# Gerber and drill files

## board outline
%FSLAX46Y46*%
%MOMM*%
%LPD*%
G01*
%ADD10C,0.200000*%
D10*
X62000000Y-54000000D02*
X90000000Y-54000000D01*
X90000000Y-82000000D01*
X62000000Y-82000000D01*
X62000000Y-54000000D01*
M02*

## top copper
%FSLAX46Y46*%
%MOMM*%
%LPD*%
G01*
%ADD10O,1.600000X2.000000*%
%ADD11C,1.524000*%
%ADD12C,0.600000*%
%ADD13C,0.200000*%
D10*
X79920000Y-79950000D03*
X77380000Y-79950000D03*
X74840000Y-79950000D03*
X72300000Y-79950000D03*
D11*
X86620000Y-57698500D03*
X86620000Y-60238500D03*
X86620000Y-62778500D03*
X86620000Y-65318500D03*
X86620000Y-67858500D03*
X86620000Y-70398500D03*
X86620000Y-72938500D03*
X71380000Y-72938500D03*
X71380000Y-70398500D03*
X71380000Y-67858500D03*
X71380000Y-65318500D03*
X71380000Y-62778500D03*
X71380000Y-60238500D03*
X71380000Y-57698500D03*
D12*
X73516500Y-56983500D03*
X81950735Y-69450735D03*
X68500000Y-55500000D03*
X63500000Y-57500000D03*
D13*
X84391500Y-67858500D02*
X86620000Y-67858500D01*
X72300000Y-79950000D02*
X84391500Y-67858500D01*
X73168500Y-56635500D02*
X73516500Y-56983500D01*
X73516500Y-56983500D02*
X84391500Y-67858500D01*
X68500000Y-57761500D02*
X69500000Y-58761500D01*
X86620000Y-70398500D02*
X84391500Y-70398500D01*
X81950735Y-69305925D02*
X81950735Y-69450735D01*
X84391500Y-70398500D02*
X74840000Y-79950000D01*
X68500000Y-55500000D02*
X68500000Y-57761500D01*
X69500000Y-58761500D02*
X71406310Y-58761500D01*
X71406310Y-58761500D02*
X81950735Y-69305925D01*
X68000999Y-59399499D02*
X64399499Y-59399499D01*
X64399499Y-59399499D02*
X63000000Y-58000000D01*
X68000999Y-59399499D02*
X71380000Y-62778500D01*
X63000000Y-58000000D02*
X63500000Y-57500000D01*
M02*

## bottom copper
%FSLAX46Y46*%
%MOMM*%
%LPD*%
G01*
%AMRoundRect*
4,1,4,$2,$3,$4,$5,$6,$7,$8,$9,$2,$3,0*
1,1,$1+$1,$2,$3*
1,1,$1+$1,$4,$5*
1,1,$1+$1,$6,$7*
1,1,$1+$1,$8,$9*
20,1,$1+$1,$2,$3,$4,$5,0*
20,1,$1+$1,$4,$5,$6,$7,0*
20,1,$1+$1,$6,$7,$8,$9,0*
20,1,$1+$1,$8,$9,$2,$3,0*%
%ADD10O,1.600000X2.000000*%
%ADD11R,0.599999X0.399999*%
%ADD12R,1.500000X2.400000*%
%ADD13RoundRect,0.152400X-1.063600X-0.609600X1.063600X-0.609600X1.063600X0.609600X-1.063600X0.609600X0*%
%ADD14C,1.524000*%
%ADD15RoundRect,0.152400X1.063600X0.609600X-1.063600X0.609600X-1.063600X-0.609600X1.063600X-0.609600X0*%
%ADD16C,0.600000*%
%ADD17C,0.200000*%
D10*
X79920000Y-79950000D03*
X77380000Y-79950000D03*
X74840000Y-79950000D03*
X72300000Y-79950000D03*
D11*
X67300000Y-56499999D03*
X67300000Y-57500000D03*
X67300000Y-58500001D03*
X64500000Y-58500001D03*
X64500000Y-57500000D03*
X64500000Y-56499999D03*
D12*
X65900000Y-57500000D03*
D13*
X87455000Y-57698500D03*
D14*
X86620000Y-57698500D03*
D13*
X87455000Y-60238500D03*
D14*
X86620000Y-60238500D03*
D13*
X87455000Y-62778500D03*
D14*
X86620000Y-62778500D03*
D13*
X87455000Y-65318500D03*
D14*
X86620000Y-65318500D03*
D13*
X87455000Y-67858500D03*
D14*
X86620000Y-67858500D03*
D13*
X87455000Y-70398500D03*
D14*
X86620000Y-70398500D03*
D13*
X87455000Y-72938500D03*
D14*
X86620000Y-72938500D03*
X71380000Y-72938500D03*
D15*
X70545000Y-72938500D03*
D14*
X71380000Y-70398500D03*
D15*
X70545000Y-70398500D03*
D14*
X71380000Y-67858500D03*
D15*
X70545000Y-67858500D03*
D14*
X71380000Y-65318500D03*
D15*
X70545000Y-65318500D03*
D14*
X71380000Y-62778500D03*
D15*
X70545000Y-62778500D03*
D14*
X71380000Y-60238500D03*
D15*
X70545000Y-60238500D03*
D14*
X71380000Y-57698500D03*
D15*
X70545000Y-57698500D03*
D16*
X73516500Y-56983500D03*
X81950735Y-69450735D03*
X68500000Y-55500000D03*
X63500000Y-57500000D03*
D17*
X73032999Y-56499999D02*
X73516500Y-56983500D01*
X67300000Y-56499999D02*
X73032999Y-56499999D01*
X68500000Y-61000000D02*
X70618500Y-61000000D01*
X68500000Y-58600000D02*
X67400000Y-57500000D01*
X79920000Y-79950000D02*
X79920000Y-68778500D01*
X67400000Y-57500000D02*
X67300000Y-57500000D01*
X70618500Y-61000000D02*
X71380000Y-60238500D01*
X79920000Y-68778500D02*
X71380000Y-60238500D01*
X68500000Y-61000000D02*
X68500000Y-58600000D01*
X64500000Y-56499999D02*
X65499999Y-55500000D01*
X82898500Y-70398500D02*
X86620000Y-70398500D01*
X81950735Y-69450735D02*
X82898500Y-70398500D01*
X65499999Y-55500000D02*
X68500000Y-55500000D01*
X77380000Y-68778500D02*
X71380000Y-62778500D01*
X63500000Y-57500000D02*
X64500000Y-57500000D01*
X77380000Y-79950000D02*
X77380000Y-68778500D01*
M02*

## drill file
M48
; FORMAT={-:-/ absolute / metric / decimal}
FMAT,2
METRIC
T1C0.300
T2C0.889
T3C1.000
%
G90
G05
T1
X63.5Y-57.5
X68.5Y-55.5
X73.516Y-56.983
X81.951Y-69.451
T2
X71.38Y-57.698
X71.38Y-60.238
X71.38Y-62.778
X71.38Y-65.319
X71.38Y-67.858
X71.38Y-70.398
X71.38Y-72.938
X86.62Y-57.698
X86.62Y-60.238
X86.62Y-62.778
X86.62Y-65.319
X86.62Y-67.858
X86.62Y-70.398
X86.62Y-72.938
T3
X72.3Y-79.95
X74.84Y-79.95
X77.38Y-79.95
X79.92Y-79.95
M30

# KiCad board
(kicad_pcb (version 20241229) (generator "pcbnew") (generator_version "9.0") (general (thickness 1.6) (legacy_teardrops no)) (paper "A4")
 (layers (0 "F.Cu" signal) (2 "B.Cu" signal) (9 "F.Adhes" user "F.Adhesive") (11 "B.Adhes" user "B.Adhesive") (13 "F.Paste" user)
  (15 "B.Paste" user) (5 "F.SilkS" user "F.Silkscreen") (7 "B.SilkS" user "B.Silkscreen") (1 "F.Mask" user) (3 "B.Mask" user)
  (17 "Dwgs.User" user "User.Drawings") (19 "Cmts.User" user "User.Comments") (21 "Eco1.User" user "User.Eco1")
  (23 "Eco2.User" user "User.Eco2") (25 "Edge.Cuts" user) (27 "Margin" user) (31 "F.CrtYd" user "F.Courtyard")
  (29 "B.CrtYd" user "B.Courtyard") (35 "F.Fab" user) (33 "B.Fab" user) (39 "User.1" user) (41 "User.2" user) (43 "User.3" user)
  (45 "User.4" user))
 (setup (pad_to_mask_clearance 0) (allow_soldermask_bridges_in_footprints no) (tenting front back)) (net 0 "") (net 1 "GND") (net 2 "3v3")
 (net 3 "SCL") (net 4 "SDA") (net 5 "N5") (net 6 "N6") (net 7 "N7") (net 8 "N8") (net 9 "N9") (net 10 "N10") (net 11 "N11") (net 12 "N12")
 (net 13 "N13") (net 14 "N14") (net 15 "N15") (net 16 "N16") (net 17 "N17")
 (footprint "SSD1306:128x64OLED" (layer "F.Cu") (at 76.3 69.35 180)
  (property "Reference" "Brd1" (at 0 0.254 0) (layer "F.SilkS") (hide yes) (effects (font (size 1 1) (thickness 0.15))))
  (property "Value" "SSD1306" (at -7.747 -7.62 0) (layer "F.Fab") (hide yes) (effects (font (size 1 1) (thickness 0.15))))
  (pad "1" thru_hole oval (at -3.62 -10.6 270) (size 2 1.6) (drill 1) (layers "*.Cu" "*.Mask") (remove_unused_layers no) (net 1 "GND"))
  (pad "2" thru_hole oval (at -1.08 -10.6 270) (size 2 1.6) (drill 1) (layers "*.Cu" "*.Mask") (remove_unused_layers no) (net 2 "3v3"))
  (pad "3" thru_hole oval (at 1.46 -10.6 270) (size 2 1.6) (drill 1) (layers "*.Cu" "*.Mask") (remove_unused_layers no) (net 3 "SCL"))
  (pad "4" thru_hole oval (at 4 -10.6 270) (size 2 1.6) (drill 1) (layers "*.Cu" "*.Mask") (remove_unused_layers no) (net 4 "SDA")))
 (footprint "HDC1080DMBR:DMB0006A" (layer "B.Cu") (at 65.9 57.5 180)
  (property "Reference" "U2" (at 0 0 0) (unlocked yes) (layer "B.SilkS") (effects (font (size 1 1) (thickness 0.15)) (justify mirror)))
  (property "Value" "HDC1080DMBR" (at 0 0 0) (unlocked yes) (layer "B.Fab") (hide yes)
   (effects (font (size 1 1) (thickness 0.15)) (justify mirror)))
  (pad "1" smd rect (at -1.4 1.000001 180) (size 0.599999 0.399999) (layers "B.Cu" "B.Mask" "B.Paste") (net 4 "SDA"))
  (pad "2" smd rect (at -1.4 0 180) (size 0.599999 0.399999) (layers "B.Cu" "B.Mask" "B.Paste") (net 1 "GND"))
  (pad "3" smd rect (at -1.4 -1.000001 180) (size 0.599999 0.399999) (layers "B.Cu" "B.Mask" "B.Paste") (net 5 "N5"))
  (pad "4" smd rect (at 1.4 -1.000001 180) (size 0.599999 0.399999) (layers "B.Cu" "B.Mask" "B.Paste") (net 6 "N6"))
  (pad "5" smd rect (at 1.4 0 180) (size 0.599999 0.399999) (layers "B.Cu" "B.Mask" "B.Paste") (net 2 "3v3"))
  (pad "6" smd rect (at 1.4 1.000001 180) (size 0.599999 0.399999) (layers "B.Cu" "B.Mask" "B.Paste") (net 3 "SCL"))
  (pad "7" smd rect (at 0 0 180) (size 1.5 2.4) (layers "B.Cu" "B.Mask") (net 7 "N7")))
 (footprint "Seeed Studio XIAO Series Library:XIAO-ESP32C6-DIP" (layer "B.Cu") (at 78.955 65.3185 180)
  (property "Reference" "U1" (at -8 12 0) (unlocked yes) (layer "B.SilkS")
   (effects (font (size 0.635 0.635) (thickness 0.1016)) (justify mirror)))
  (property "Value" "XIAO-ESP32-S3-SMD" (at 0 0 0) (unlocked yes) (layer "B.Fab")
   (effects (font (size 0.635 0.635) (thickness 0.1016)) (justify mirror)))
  (pad "1" smd roundrect (at -8.5 7.62) (size 2.432 1.524) (layers "B.Cu" "B.Mask") (roundrect_rratio 0.1) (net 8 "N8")
   (thermal_bridge_angle 45))
  (pad "1" thru_hole circle (at -7.665 7.62) (size 1.524 1.524) (drill 0.889) (layers "*.Cu" "*.Mask") (remove_unused_layers no)
   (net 8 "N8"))
  (pad "2" smd roundrect (at -8.5 5.08) (size 2.432 1.524) (layers "B.Cu" "B.Mask") (roundrect_rratio 0.1) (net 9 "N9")
   (thermal_bridge_angle 45))
  (pad "2" thru_hole circle (at -7.665 5.08) (size 1.524 1.524) (drill 0.889) (layers "*.Cu" "*.Mask") (remove_unused_layers no)
   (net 9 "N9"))
  (pad "3" smd roundrect (at -8.5 2.54) (size 2.432 1.524) (layers "B.Cu" "B.Mask") (roundrect_rratio 0.1) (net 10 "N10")
   (thermal_bridge_angle 45))
  (pad "3" thru_hole circle (at -7.665 2.54) (size 1.524 1.524) (drill 0.889) (layers "*.Cu" "*.Mask") (remove_unused_layers no)
   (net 10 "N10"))
  (pad "4" smd roundrect (at -8.5 0) (size 2.432 1.524) (layers "B.Cu" "B.Mask") (roundrect_rratio 0.1) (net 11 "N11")
   (thermal_bridge_angle 45))
  (pad "4" thru_hole circle (at -7.665 0) (size 1.524 1.524) (drill 0.889) (layers "*.Cu" "*.Mask") (remove_unused_layers no) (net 11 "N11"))
  (pad "5" smd roundrect (at -8.5 -2.54) (size 2.432 1.524) (layers "B.Cu" "B.Mask") (roundrect_rratio 0.1) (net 4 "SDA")
   (thermal_bridge_angle 45))
  (pad "5" thru_hole circle (at -7.665 -2.54) (size 1.524 1.524) (drill 0.889) (layers "*.Cu" "*.Mask") (remove_unused_layers no)
   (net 4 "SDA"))
  (pad "6" smd roundrect (at -8.5 -5.08) (size 2.432 1.524) (layers "B.Cu" "B.Mask") (roundrect_rratio 0.1) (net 3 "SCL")
   (thermal_bridge_angle 45))
  (pad "6" thru_hole circle (at -7.665 -5.08) (size 1.524 1.524) (drill 0.889) (layers "*.Cu" "*.Mask") (remove_unused_layers no)
   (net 3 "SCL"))
  (pad "7" smd roundrect (at -8.5 -7.62) (size 2.432 1.524) (layers "B.Cu" "B.Mask") (roundrect_rratio 0.1) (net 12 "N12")
   (thermal_bridge_angle 45))
  (pad "7" thru_hole circle (at -7.665 -7.62) (size 1.524 1.524) (drill 0.889) (layers "*.Cu" "*.Mask") (remove_unused_layers no)
   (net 12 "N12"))
  (pad "8" thru_hole circle (at 7.575 -7.62 180) (size 1.524 1.524) (drill 0.889) (layers "*.Cu" "*.Mask") (remove_unused_layers no)
   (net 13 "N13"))
  (pad "8" smd roundrect (at 8.41 -7.62 180) (size 2.432 1.524) (layers "B.Cu" "B.Mask") (roundrect_rratio 0.1) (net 13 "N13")
   (thermal_bridge_angle 45))
  (pad "9" thru_hole circle (at 7.575 -5.08 180) (size 1.524 1.524) (drill 0.889) (layers "*.Cu" "*.Mask") (remove_unused_layers no)
   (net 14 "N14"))
  (pad "9" smd roundrect (at 8.41 -5.08 180) (size 2.432 1.524) (layers "B.Cu" "B.Mask") (roundrect_rratio 0.1) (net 14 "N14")
   (thermal_bridge_angle 45))
  (pad "10" thru_hole circle (at 7.575 -2.54 180) (size 1.524 1.524) (drill 0.889) (layers "*.Cu" "*.Mask") (remove_unused_layers no)
   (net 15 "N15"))
  (pad "10" smd roundrect (at 8.41 -2.54 180) (size 2.432 1.524) (layers "B.Cu" "B.Mask") (roundrect_rratio 0.1) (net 15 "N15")
   (thermal_bridge_angle 45))
  (pad "11" thru_hole circle (at 7.575 0 180) (size 1.524 1.524) (drill 0.889) (layers "*.Cu" "*.Mask") (remove_unused_layers no)
   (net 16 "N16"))
  (pad "11" smd roundrect (at 8.41 0 180) (size 2.432 1.524) (layers "B.Cu" "B.Mask") (roundrect_rratio 0.1) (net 16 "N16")
   (thermal_bridge_angle 45))
  (pad "12" thru_hole circle (at 7.575 2.54 180) (size 1.524 1.524) (drill 0.889) (layers "*.Cu" "*.Mask") (remove_unused_layers no)
   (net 2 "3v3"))
  (pad "12" smd roundrect (at 8.41 2.54 180) (size 2.432 1.524) (layers "B.Cu" "B.Mask") (roundrect_rratio 0.1) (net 2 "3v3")
   (thermal_bridge_angle 45))
  (pad "13" thru_hole circle (at 7.575 5.08 180) (size 1.524 1.524) (drill 0.889) (layers "*.Cu" "*.Mask") (remove_unused_layers no)
   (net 1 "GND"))
  (pad "13" smd roundrect (at 8.41 5.08 180) (size 2.432 1.524) (layers "B.Cu" "B.Mask") (roundrect_rratio 0.1) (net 1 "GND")
   (thermal_bridge_angle 45))
  (pad "14" thru_hole circle (at 7.575 7.62 180) (size 1.524 1.524) (drill 0.889) (layers "*.Cu" "*.Mask") (remove_unused_layers no)
   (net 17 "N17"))
  (pad "14" smd roundrect (at 8.41 7.62 180) (size 2.432 1.524) (layers "B.Cu" "B.Mask") (roundrect_rratio 0.1) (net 17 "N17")
   (thermal_bridge_angle 45)))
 (gr_rect (start 62 54) (end 90 82) (stroke (width 0.2) (type solid)) (fill no) (layer "Edge.Cuts"))
 (segment (start 84.3915 67.8585) (end 86.62 67.8585) (width 0.2) (layer "F.Cu") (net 4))
 (segment (start 72.3 79.95) (end 84.3915 67.8585) (width 0.2) (layer "F.Cu") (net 4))
 (segment (start 73.1685 56.6355) (end 73.5165 56.9835) (width 0.2) (layer "F.Cu") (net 4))
 (segment (start 73.5165 56.9835) (end 84.3915 67.8585) (width 0.2) (layer "F.Cu") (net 4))
 (via (at 73.5165 56.9835) (size 0.6) (drill 0.3) (layers "F.Cu" "B.Cu") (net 4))
 (segment (start 73.032999 56.499999) (end 73.5165 56.9835) (width 0.2) (layer "B.Cu") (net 4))
 (segment (start 67.3 56.499999) (end 73.032999 56.499999) (width 0.2) (layer "B.Cu") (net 4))
 (segment (start 68.5 61) (end 70.6185 61) (width 0.2) (layer "B.Cu") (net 1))
 (segment (start 68.5 58.6) (end 67.4 57.5) (width 0.2) (layer "B.Cu") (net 1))
 (segment (start 79.92 79.95) (end 79.92 68.7785) (width 0.2) (layer "B.Cu") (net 1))
 (segment (start 67.4 57.5) (end 67.3 57.5) (width 0.2) (layer "B.Cu") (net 1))
 (segment (start 70.6185 61) (end 71.38 60.2385) (width 0.2) (layer "B.Cu") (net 1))
 (segment (start 79.92 68.7785) (end 71.38 60.2385) (width 0.2) (layer "B.Cu") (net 1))
 (segment (start 68.5 61) (end 68.5 58.6) (width 0.2) (layer "B.Cu") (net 1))
 (segment (start 68.5 57.7615) (end 69.5 58.7615) (width 0.2) (layer "F.Cu") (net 3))
 (segment (start 86.62 70.3985) (end 84.3915 70.3985) (width 0.2) (layer "F.Cu") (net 3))
 (segment (start 81.950735 69.305925) (end 81.950735 69.450735) (width 0.2) (layer "F.Cu") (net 3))
 (segment (start 84.3915 70.3985) (end 74.84 79.95) (width 0.2) (layer "F.Cu") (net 3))
 (segment (start 68.5 55.5) (end 68.5 57.7615) (width 0.2) (layer "F.Cu") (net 3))
 (segment (start 69.5 58.7615) (end 71.40631 58.7615) (width 0.2) (layer "F.Cu") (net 3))
 (segment (start 71.40631 58.7615) (end 81.950735 69.305925) (width 0.2) (layer "F.Cu") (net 3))
 (via (at 81.950735 69.450735) (size 0.6) (drill 0.3) (layers "F.Cu" "B.Cu") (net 3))
 (via (at 68.5 55.5) (size 0.6) (drill 0.3) (layers "F.Cu" "B.Cu") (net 3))
 (segment (start 64.5 56.499999) (end 65.499999 55.5) (width 0.2) (layer "B.Cu") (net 3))
 (segment (start 82.8985 70.3985) (end 86.62 70.3985) (width 0.2) (layer "B.Cu") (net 3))
 (segment (start 81.950735 69.450735) (end 82.8985 70.3985) (width 0.2) (layer "B.Cu") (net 3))
 (segment (start 65.499999 55.5) (end 68.5 55.5) (width 0.2) (layer "B.Cu") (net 3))
 (segment (start 68.000999 59.399499) (end 64.399499 59.399499) (width 0.2) (layer "F.Cu") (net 2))
 (segment (start 64.399499 59.399499) (end 63 58) (width 0.2) (layer "F.Cu") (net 2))
 (segment (start 68.000999 59.399499) (end 71.38 62.7785) (width 0.2) (layer "F.Cu") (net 2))
 (segment (start 63 58) (end 63.5 57.5) (width 0.2) (layer "F.Cu") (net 2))
 (via (at 63.5 57.5) (size 0.6) (drill 0.3) (layers "F.Cu" "B.Cu") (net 2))
 (segment (start 77.38 68.7785) (end 71.38 62.7785) (width 0.2) (layer "B.Cu") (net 2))
 (segment (start 63.5 57.5) (end 64.5 57.5) (width 0.2) (layer "B.Cu") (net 2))
 (segment (start 77.38 79.95) (end 77.38 68.7785) (width 0.2) (layer "B.Cu") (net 2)))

